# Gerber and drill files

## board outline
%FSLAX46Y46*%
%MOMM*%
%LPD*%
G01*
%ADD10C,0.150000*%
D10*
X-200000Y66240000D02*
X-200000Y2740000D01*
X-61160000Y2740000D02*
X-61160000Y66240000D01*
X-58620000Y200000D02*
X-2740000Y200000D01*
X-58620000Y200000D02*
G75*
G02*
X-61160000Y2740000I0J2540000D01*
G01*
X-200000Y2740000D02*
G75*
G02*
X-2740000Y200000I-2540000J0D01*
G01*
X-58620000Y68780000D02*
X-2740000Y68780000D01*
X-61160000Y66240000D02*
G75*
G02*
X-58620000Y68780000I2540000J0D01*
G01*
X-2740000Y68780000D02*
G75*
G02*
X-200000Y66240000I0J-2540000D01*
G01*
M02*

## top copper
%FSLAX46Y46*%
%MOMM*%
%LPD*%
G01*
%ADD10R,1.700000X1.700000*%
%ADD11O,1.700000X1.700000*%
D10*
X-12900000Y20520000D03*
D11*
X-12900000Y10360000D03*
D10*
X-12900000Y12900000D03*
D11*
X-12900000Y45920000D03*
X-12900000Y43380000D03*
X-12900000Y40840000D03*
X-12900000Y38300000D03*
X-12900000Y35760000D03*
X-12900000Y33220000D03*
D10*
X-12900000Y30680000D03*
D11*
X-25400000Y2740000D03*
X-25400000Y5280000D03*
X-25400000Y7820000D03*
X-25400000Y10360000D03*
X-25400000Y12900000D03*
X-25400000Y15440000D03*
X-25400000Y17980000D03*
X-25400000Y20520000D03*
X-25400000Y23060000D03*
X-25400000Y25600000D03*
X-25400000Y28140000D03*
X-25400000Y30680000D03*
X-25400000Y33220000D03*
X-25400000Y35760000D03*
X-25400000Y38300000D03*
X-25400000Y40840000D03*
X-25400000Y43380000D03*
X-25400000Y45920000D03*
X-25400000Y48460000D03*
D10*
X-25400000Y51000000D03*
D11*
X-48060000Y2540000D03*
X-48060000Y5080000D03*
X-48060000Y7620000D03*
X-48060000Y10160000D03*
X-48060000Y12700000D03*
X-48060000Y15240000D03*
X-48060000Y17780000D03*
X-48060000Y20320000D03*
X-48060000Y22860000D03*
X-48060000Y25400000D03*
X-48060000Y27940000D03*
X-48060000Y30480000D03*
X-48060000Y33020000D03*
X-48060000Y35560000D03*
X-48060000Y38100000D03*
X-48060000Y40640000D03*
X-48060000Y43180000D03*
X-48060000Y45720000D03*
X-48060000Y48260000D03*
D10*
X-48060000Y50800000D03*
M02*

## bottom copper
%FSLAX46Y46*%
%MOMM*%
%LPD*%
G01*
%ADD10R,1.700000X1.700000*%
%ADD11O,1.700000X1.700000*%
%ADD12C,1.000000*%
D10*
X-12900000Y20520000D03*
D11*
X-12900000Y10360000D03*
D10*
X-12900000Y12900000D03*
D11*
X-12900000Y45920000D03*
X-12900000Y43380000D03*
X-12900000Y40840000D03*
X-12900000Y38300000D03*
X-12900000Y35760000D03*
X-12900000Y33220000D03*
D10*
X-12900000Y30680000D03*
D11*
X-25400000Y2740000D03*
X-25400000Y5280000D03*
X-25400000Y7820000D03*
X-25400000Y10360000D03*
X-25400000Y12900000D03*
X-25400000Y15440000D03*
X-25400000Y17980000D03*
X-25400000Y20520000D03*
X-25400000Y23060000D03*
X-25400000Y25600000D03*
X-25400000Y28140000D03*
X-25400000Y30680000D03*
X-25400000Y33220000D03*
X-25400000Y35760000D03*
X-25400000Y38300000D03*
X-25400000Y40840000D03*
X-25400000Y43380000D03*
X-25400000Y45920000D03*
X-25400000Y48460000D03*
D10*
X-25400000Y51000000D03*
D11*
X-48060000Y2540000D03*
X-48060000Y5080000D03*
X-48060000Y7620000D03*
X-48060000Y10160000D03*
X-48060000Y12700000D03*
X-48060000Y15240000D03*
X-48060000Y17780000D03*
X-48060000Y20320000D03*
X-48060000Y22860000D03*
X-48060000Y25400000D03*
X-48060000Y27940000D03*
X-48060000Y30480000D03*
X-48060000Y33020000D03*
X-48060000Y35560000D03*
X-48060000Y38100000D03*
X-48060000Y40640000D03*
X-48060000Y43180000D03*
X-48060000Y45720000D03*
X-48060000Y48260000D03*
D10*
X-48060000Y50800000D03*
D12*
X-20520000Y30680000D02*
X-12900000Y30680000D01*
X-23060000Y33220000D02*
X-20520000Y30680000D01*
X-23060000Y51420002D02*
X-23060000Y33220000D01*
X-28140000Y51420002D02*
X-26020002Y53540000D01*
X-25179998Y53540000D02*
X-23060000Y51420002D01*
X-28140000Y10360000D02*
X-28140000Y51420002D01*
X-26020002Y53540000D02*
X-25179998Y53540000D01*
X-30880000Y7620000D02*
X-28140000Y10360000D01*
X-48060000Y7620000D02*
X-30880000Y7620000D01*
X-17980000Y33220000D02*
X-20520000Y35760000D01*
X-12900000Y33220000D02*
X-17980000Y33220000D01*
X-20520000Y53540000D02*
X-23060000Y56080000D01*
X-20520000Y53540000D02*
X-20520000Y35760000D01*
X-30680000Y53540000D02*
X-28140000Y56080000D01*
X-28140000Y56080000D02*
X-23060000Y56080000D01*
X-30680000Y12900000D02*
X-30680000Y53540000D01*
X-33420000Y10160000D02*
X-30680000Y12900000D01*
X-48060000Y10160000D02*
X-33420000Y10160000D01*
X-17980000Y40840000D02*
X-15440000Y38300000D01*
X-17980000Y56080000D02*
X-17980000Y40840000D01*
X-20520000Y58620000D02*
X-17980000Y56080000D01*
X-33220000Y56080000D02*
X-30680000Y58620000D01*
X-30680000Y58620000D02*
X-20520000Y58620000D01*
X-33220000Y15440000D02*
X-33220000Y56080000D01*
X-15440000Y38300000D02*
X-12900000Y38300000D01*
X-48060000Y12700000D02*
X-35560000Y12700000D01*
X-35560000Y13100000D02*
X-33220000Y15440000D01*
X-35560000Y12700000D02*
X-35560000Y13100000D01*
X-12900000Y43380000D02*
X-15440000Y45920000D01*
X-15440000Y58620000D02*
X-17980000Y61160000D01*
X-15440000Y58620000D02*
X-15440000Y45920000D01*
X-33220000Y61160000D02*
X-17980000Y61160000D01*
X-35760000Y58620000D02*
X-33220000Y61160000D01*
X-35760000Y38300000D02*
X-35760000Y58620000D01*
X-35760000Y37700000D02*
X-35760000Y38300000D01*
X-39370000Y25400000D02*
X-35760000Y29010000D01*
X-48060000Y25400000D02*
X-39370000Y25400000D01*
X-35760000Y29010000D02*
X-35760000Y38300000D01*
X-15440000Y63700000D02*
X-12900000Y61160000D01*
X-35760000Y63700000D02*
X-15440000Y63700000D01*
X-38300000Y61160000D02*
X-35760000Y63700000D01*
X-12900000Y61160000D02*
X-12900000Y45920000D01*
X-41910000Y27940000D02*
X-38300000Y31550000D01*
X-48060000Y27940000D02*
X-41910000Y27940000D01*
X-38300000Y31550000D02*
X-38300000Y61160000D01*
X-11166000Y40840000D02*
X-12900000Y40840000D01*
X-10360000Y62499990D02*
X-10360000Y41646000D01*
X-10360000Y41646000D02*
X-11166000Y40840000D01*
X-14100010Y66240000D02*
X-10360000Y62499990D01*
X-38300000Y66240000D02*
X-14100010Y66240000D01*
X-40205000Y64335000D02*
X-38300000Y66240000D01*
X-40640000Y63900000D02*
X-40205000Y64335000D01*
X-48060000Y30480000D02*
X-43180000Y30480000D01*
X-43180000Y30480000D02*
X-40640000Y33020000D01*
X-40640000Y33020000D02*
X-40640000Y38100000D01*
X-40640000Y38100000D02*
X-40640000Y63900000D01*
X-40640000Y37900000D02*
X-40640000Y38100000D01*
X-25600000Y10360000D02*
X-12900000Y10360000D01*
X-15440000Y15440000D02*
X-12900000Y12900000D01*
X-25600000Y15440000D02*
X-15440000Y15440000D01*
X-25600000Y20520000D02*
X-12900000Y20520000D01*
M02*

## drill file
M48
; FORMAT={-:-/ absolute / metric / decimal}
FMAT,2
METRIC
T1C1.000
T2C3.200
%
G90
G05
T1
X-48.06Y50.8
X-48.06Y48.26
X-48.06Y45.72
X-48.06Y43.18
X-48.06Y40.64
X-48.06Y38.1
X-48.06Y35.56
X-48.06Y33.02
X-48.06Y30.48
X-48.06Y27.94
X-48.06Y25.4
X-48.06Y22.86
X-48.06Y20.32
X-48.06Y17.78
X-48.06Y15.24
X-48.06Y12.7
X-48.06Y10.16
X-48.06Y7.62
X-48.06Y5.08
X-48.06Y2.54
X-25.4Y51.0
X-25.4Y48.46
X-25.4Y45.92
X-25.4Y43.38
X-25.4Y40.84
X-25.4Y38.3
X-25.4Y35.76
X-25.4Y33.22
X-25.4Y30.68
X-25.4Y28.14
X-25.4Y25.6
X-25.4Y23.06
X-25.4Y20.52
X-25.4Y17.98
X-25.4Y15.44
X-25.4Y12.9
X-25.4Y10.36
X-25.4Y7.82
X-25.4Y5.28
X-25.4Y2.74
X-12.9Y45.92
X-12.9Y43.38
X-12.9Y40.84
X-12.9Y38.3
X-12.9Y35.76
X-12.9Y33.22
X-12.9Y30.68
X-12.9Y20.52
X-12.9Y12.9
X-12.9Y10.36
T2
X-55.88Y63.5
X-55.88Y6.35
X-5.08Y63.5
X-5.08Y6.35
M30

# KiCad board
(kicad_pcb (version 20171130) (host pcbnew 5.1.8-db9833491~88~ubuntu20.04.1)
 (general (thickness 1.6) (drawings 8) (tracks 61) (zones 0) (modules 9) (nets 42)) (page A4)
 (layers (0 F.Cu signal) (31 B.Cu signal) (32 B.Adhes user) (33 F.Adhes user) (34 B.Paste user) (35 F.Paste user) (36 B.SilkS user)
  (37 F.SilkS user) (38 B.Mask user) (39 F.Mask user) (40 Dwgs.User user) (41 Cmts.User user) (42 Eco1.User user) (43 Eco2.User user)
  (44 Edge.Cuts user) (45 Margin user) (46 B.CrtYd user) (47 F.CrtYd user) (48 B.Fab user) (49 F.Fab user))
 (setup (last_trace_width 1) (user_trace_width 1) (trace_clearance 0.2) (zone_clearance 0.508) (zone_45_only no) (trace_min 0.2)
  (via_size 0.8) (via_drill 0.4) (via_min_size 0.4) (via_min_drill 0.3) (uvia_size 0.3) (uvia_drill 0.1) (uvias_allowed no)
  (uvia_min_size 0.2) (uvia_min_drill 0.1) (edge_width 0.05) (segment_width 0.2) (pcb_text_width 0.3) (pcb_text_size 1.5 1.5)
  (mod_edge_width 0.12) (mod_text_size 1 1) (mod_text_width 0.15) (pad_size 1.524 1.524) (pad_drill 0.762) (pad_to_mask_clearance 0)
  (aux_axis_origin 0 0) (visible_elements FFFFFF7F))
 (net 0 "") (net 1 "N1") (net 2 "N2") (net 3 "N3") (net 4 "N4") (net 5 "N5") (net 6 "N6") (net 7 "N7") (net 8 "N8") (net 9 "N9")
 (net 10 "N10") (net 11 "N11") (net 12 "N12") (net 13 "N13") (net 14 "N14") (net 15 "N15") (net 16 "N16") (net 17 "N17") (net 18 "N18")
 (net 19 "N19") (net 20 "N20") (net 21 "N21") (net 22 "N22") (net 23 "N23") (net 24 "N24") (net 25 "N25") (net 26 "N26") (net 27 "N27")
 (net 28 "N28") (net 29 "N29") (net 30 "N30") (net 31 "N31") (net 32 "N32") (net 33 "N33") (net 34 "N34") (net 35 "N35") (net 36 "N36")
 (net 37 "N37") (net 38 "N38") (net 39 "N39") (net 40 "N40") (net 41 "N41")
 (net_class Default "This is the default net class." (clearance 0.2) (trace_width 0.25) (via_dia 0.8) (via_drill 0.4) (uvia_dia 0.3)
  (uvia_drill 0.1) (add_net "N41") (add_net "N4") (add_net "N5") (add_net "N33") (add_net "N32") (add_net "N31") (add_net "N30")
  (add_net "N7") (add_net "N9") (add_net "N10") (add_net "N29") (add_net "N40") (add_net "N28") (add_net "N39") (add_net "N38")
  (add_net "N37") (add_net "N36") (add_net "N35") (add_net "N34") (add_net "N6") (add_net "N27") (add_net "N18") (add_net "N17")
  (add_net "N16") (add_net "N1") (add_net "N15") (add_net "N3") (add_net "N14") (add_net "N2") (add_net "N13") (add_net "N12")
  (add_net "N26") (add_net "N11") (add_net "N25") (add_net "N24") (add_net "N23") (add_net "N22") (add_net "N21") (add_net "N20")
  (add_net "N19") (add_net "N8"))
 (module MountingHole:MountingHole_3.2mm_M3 (layer F.Cu) (at -5.08 -6.35)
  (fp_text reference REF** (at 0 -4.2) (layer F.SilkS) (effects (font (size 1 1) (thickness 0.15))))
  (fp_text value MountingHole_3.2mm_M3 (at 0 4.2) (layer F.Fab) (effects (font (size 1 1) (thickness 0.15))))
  (pad 1 np_thru_hole circle (at 0 0) (size 3.2 3.2) (drill 3.2) (layers *.Cu *.Mask)))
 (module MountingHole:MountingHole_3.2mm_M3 (layer F.Cu) (at -55.88 -6.35)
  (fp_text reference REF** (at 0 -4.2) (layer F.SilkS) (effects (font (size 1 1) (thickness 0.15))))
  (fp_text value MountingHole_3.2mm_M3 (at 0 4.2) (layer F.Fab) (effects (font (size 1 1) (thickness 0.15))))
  (pad 1 np_thru_hole circle (at 0 0) (size 3.2 3.2) (drill 3.2) (layers *.Cu *.Mask)))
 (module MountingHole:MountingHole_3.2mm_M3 (layer F.Cu) (at -55.88 -63.5)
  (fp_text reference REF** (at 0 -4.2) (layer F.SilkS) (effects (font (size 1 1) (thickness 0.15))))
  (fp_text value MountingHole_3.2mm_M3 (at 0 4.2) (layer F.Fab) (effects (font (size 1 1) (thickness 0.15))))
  (pad 1 np_thru_hole circle (at 0 0) (size 3.2 3.2) (drill 3.2) (layers *.Cu *.Mask)))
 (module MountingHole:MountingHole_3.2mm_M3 (layer F.Cu) (at -5.08 -63.5)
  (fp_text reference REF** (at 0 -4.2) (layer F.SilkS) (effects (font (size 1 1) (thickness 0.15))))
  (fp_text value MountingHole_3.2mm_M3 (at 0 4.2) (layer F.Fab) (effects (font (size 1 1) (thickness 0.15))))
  (pad 1 np_thru_hole circle (at 0 0) (size 3.2 3.2) (drill 3.2) (layers *.Cu *.Mask)))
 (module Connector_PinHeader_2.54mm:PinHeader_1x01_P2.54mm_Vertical (layer F.Cu) (at -12.9 -20.52)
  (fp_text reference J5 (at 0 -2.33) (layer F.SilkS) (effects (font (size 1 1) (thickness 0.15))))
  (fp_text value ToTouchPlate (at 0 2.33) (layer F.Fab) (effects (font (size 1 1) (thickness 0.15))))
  (pad 1 thru_hole rect (at 0 0) (size 1.7 1.7) (drill 1) (layers *.Cu *.Mask) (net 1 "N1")))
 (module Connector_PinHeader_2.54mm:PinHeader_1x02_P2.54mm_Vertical (layer F.Cu) (at -12.9 -12.9)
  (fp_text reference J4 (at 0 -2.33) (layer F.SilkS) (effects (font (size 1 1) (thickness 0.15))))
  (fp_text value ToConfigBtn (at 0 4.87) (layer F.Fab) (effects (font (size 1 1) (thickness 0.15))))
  (pad 2 thru_hole oval (at 0 2.54) (size 1.7 1.7) (drill 1) (layers *.Cu *.Mask) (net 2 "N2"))
  (pad 1 thru_hole rect (at 0 0) (size 1.7 1.7) (drill 1) (layers *.Cu *.Mask) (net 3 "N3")))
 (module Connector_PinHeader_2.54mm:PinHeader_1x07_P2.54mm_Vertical (layer F.Cu) (at -12.9 -30.68 180)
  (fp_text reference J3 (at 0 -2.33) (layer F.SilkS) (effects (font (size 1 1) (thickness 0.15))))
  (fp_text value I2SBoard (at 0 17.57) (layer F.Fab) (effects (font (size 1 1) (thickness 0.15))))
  (pad 7 thru_hole oval (at 0 15.24 180) (size 1.7 1.7) (drill 1) (layers *.Cu *.Mask) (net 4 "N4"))
  (pad 6 thru_hole oval (at 0 12.7 180) (size 1.7 1.7) (drill 1) (layers *.Cu *.Mask) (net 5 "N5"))
  (pad 5 thru_hole oval (at 0 10.16 180) (size 1.7 1.7) (drill 1) (layers *.Cu *.Mask) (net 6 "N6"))
  (pad 4 thru_hole oval (at 0 7.62 180) (size 1.7 1.7) (drill 1) (layers *.Cu *.Mask) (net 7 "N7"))
  (pad 3 thru_hole oval (at 0 5.08 180) (size 1.7 1.7) (drill 1) (layers *.Cu *.Mask) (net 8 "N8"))
  (pad 2 thru_hole oval (at 0 2.54 180) (size 1.7 1.7) (drill 1) (layers *.Cu *.Mask) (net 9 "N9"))
  (pad 1 thru_hole rect (at 0 0 180) (size 1.7 1.7) (drill 1) (layers *.Cu *.Mask) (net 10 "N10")))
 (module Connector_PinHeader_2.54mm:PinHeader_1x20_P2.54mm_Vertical (layer F.Cu) (at -25.4 -51)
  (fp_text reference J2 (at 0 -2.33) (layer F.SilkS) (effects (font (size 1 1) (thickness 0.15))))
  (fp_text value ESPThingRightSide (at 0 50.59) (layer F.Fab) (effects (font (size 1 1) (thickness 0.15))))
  (pad 20 thru_hole oval (at 0 48.26) (size 1.7 1.7) (drill 1) (layers *.Cu *.Mask) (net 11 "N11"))
  (pad 19 thru_hole oval (at 0 45.72) (size 1.7 1.7) (drill 1) (layers *.Cu *.Mask) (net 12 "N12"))
  (pad 18 thru_hole oval (at 0 43.18) (size 1.7 1.7) (drill 1) (layers *.Cu *.Mask) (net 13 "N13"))
  (pad 17 thru_hole oval (at 0 40.64) (size 1.7 1.7) (drill 1) (layers *.Cu *.Mask) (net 2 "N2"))
  (pad 16 thru_hole oval (at 0 38.1) (size 1.7 1.7) (drill 1) (layers *.Cu *.Mask) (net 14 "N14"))
  (pad 15 thru_hole oval (at 0 35.56) (size 1.7 1.7) (drill 1) (layers *.Cu *.Mask) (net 3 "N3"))
  (pad 14 thru_hole oval (at 0 33.02) (size 1.7 1.7) (drill 1) (layers *.Cu *.Mask) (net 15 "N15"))
  (pad 13 thru_hole oval (at 0 30.48) (size 1.7 1.7) (drill 1) (layers *.Cu *.Mask) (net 1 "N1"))
  (pad 12 thru_hole oval (at 0 27.94) (size 1.7 1.7) (drill 1) (layers *.Cu *.Mask) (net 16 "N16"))
  (pad 11 thru_hole oval (at 0 25.4) (size 1.7 1.7) (drill 1) (layers *.Cu *.Mask) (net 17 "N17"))
  (pad 10 thru_hole oval (at 0 22.86) (size 1.7 1.7) (drill 1) (layers *.Cu *.Mask) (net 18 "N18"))
  (pad 9 thru_hole oval (at 0 20.32) (size 1.7 1.7) (drill 1) (layers *.Cu *.Mask) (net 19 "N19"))
  (pad 8 thru_hole oval (at 0 17.78) (size 1.7 1.7) (drill 1) (layers *.Cu *.Mask) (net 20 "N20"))
  (pad 7 thru_hole oval (at 0 15.24) (size 1.7 1.7) (drill 1) (layers *.Cu *.Mask) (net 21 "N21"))
  (pad 6 thru_hole oval (at 0 12.7) (size 1.7 1.7) (drill 1) (layers *.Cu *.Mask) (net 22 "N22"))
  (pad 5 thru_hole oval (at 0 10.16) (size 1.7 1.7) (drill 1) (layers *.Cu *.Mask) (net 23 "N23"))
  (pad 4 thru_hole oval (at 0 7.62) (size 1.7 1.7) (drill 1) (layers *.Cu *.Mask) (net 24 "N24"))
  (pad 3 thru_hole oval (at 0 5.08) (size 1.7 1.7) (drill 1) (layers *.Cu *.Mask) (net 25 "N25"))
  (pad 2 thru_hole oval (at 0 2.54) (size 1.7 1.7) (drill 1) (layers *.Cu *.Mask) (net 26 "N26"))
  (pad 1 thru_hole rect (at 0 0) (size 1.7 1.7) (drill 1) (layers *.Cu *.Mask) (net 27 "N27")))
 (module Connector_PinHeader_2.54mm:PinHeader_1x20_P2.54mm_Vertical (layer F.Cu) (at -48.06 -50.8)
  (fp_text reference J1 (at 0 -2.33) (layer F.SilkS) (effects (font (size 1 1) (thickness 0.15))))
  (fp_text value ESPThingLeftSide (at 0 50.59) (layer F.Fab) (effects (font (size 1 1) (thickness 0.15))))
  (pad 20 thru_hole oval (at 0 48.26) (size 1.7 1.7) (drill 1) (layers *.Cu *.Mask) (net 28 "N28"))
  (pad 19 thru_hole oval (at 0 45.72) (size 1.7 1.7) (drill 1) (layers *.Cu *.Mask) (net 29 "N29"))
  (pad 18 thru_hole oval (at 0 43.18) (size 1.7 1.7) (drill 1) (layers *.Cu *.Mask) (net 10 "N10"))
  (pad 17 thru_hole oval (at 0 40.64) (size 1.7 1.7) (drill 1) (layers *.Cu *.Mask) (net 9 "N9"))
  (pad 16 thru_hole oval (at 0 38.1) (size 1.7 1.7) (drill 1) (layers *.Cu *.Mask) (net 7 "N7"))
  (pad 15 thru_hole oval (at 0 35.56) (size 1.7 1.7) (drill 1) (layers *.Cu *.Mask) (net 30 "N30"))
  (pad 14 thru_hole oval (at 0 33.02) (size 1.7 1.7) (drill 1) (layers *.Cu *.Mask) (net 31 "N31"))
  (pad 13 thru_hole oval (at 0 30.48) (size 1.7 1.7) (drill 1) (layers *.Cu *.Mask) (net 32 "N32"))
  (pad 12 thru_hole oval (at 0 27.94) (size 1.7 1.7) (drill 1) (layers *.Cu *.Mask) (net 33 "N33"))
  (pad 11 thru_hole oval (at 0 25.4) (size 1.7 1.7) (drill 1) (layers *.Cu *.Mask) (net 5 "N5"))
  (pad 10 thru_hole oval (at 0 22.86) (size 1.7 1.7) (drill 1) (layers *.Cu *.Mask) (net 4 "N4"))
  (pad 9 thru_hole oval (at 0 20.32) (size 1.7 1.7) (drill 1) (layers *.Cu *.Mask) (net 6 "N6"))
  (pad 8 thru_hole oval (at 0 17.78) (size 1.7 1.7) (drill 1) (layers *.Cu *.Mask) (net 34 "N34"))
  (pad 7 thru_hole oval (at 0 15.24) (size 1.7 1.7) (drill 1) (layers *.Cu *.Mask) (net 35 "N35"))
  (pad 6 thru_hole oval (at 0 12.7) (size 1.7 1.7) (drill 1) (layers *.Cu *.Mask) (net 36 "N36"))
  (pad 5 thru_hole oval (at 0 10.16) (size 1.7 1.7) (drill 1) (layers *.Cu *.Mask) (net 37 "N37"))
  (pad 4 thru_hole oval (at 0 7.62) (size 1.7 1.7) (drill 1) (layers *.Cu *.Mask) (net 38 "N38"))
  (pad 3 thru_hole oval (at 0 5.08) (size 1.7 1.7) (drill 1) (layers *.Cu *.Mask) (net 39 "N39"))
  (pad 2 thru_hole oval (at 0 2.54) (size 1.7 1.7) (drill 1) (layers *.Cu *.Mask) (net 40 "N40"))
  (pad 1 thru_hole rect (at 0 0) (size 1.7 1.7) (drill 1) (layers *.Cu *.Mask) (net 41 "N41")))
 (gr_line (start -0.2 -66.24) (end -0.2 -2.74) (layer Edge.Cuts) (width 0.15))
 (gr_line (start -61.16 -2.74) (end -61.16 -66.24) (layer Edge.Cuts) (width 0.15))
 (gr_line (start -58.62 -0.2) (end -2.74 -0.2) (layer Edge.Cuts) (width 0.15))
 (gr_arc (start -58.62 -2.74) (end -61.16 -2.74) (angle -90) (layer Edge.Cuts) (width 0.15))
 (gr_arc (start -2.74 -2.74) (end -2.74 -0.2) (angle -90) (layer Edge.Cuts) (width 0.15))
 (gr_line (start -58.62 -68.78) (end -2.74 -68.78) (layer Edge.Cuts) (width 0.15))
 (gr_arc (start -58.62 -66.24) (end -58.62 -68.78) (angle -90) (layer Edge.Cuts) (width 0.15))
 (gr_arc (start -2.74 -66.24) (end -0.2 -66.24) (angle -90) (layer Edge.Cuts) (width 0.15))
 (segment (start -20.52 -30.68) (end -12.9 -30.68) (width 1) (layer B.Cu) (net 10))
 (segment (start -23.06 -33.22) (end -20.52 -30.68) (width 1) (layer B.Cu) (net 10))
 (segment (start -23.06 -51.420002) (end -23.06 -33.22) (width 1) (layer B.Cu) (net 10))
 (segment (start -28.14 -51.420002) (end -26.020002 -53.54) (width 1) (layer B.Cu) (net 10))
 (segment (start -25.179998 -53.54) (end -23.06 -51.420002) (width 1) (layer B.Cu) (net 10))
 (segment (start -28.14 -10.36) (end -28.14 -51.420002) (width 1) (layer B.Cu) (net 10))
 (segment (start -26.020002 -53.54) (end -25.179998 -53.54) (width 1) (layer B.Cu) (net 10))
 (segment (start -30.88 -7.62) (end -28.14 -10.36) (width 1) (layer B.Cu) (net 10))
 (segment (start -48.06 -7.62) (end -30.88 -7.62) (width 1) (layer B.Cu) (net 10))
 (segment (start -17.98 -33.22) (end -20.52 -35.76) (width 1) (layer B.Cu) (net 9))
 (segment (start -12.9 -33.22) (end -17.98 -33.22) (width 1) (layer B.Cu) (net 9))
 (segment (start -20.52 -53.54) (end -23.06 -56.08) (width 1) (layer B.Cu) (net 9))
 (segment (start -20.52 -53.54) (end -20.52 -35.76) (width 1) (layer B.Cu) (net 9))
 (segment (start -30.68 -53.54) (end -28.14 -56.08) (width 1) (layer B.Cu) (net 9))
 (segment (start -28.14 -56.08) (end -23.06 -56.08) (width 1) (layer B.Cu) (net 9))
 (segment (start -30.68 -12.9) (end -30.68 -53.54) (width 1) (layer B.Cu) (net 9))
 (segment (start -33.42 -10.16) (end -30.68 -12.9) (width 1) (layer B.Cu) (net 9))
 (segment (start -48.06 -10.16) (end -33.42 -10.16) (width 1) (layer B.Cu) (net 9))
 (segment (start -17.98 -40.84) (end -15.44 -38.3) (width 1) (layer B.Cu) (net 7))
 (segment (start -17.98 -56.08) (end -17.98 -40.84) (width 1) (layer B.Cu) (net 7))
 (segment (start -20.52 -58.62) (end -17.98 -56.08) (width 1) (layer B.Cu) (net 7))
 (segment (start -33.22 -56.08) (end -30.68 -58.62) (width 1) (layer B.Cu) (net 7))
 (segment (start -30.68 -58.62) (end -20.52 -58.62) (width 1) (layer B.Cu) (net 7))
 (segment (start -33.22 -15.44) (end -33.22 -56.08) (width 1) (layer B.Cu) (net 7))
 (segment (start -15.44 -38.3) (end -12.9 -38.3) (width 1) (layer B.Cu) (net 7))
 (segment (start -48.06 -12.7) (end -35.56 -12.7) (width 1) (layer B.Cu) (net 7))
 (segment (start -35.56 -13.1) (end -33.22 -15.44) (width 1) (layer B.Cu) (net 7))
 (segment (start -35.56 -12.7) (end -35.56 -13.1) (width 1) (layer B.Cu) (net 7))
 (segment (start -12.9 -43.38) (end -15.44 -45.92) (width 1) (layer B.Cu) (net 5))
 (segment (start -15.44 -58.62) (end -17.98 -61.16) (width 1) (layer B.Cu) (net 5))
 (segment (start -15.44 -58.62) (end -15.44 -45.92) (width 1) (layer B.Cu) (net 5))
 (segment (start -33.22 -61.16) (end -17.98 -61.16) (width 1) (layer B.Cu) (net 5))
 (segment (start -35.76 -58.62) (end -33.22 -61.16) (width 1) (layer B.Cu) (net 5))
 (segment (start -35.76 -38.3) (end -35.76 -58.62) (width 1) (layer B.Cu) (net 5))
 (segment (start -35.76 -37.7) (end -35.76 -38.3) (width 1) (layer B.Cu) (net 5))
 (segment (start -39.37 -25.4) (end -35.76 -29.01) (width 1) (layer B.Cu) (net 5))
 (segment (start -48.06 -25.4) (end -39.37 -25.4) (width 1) (layer B.Cu) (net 5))
 (segment (start -35.76 -29.01) (end -35.76 -38.3) (width 1) (layer B.Cu) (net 5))
 (segment (start -15.44 -63.7) (end -12.9 -61.16) (width 1) (layer B.Cu) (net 4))
 (segment (start -35.76 -63.7) (end -15.44 -63.7) (width 1) (layer B.Cu) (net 4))
 (segment (start -38.3 -61.16) (end -35.76 -63.7) (width 1) (layer B.Cu) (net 4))
 (segment (start -12.9 -61.16) (end -12.9 -45.92) (width 1) (layer B.Cu) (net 4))
 (segment (start -41.91 -27.94) (end -38.3 -31.55) (width 1) (layer B.Cu) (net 4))
 (segment (start -48.06 -27.94) (end -41.91 -27.94) (width 1) (layer B.Cu) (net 4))
 (segment (start -38.3 -31.55) (end -38.3 -61.16) (width 1) (layer B.Cu) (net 4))
 (segment (start -11.166 -40.84) (end -12.9 -40.84) (width 1) (layer B.Cu) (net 6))
 (segment (start -10.36 -62.49999) (end -10.36 -41.646) (width 1) (layer B.Cu) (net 6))
 (segment (start -10.36 -41.646) (end -11.166 -40.84) (width 1) (layer B.Cu) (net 6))
 (segment (start -14.10001 -66.24) (end -10.36 -62.49999) (width 1) (layer B.Cu) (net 6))
 (segment (start -38.3 -66.24) (end -14.10001 -66.24) (width 1) (layer B.Cu) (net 6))
 (segment (start -40.205 -64.335) (end -38.3 -66.24) (width 1) (layer B.Cu) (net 6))
 (segment (start -40.64 -63.9) (end -40.205 -64.335) (width 1) (layer B.Cu) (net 6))
 (segment (start -48.06 -30.48) (end -43.18 -30.48) (width 1) (layer B.Cu) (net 6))
 (segment (start -43.18 -30.48) (end -40.64 -33.02) (width 1) (layer B.Cu) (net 6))
 (segment (start -40.64 -33.02) (end -40.64 -38.1) (width 1) (layer B.Cu) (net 6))
 (segment (start -40.64 -38.1) (end -40.64 -63.9) (width 1) (layer B.Cu) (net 6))
 (segment (start -40.64 -37.9) (end -40.64 -38.1) (width 1) (layer B.Cu) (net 6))
 (segment (start -25.6 -10.36) (end -12.9 -10.36) (width 1) (layer B.Cu) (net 2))
 (segment (start -15.44 -15.44) (end -12.9 -12.9) (width 1) (layer B.Cu) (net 3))
 (segment (start -25.6 -15.44) (end -15.44 -15.44) (width 1) (layer B.Cu) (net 3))
 (segment (start -25.6 -20.52) (end -12.9 -20.52) (width 1) (layer B.Cu) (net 1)))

